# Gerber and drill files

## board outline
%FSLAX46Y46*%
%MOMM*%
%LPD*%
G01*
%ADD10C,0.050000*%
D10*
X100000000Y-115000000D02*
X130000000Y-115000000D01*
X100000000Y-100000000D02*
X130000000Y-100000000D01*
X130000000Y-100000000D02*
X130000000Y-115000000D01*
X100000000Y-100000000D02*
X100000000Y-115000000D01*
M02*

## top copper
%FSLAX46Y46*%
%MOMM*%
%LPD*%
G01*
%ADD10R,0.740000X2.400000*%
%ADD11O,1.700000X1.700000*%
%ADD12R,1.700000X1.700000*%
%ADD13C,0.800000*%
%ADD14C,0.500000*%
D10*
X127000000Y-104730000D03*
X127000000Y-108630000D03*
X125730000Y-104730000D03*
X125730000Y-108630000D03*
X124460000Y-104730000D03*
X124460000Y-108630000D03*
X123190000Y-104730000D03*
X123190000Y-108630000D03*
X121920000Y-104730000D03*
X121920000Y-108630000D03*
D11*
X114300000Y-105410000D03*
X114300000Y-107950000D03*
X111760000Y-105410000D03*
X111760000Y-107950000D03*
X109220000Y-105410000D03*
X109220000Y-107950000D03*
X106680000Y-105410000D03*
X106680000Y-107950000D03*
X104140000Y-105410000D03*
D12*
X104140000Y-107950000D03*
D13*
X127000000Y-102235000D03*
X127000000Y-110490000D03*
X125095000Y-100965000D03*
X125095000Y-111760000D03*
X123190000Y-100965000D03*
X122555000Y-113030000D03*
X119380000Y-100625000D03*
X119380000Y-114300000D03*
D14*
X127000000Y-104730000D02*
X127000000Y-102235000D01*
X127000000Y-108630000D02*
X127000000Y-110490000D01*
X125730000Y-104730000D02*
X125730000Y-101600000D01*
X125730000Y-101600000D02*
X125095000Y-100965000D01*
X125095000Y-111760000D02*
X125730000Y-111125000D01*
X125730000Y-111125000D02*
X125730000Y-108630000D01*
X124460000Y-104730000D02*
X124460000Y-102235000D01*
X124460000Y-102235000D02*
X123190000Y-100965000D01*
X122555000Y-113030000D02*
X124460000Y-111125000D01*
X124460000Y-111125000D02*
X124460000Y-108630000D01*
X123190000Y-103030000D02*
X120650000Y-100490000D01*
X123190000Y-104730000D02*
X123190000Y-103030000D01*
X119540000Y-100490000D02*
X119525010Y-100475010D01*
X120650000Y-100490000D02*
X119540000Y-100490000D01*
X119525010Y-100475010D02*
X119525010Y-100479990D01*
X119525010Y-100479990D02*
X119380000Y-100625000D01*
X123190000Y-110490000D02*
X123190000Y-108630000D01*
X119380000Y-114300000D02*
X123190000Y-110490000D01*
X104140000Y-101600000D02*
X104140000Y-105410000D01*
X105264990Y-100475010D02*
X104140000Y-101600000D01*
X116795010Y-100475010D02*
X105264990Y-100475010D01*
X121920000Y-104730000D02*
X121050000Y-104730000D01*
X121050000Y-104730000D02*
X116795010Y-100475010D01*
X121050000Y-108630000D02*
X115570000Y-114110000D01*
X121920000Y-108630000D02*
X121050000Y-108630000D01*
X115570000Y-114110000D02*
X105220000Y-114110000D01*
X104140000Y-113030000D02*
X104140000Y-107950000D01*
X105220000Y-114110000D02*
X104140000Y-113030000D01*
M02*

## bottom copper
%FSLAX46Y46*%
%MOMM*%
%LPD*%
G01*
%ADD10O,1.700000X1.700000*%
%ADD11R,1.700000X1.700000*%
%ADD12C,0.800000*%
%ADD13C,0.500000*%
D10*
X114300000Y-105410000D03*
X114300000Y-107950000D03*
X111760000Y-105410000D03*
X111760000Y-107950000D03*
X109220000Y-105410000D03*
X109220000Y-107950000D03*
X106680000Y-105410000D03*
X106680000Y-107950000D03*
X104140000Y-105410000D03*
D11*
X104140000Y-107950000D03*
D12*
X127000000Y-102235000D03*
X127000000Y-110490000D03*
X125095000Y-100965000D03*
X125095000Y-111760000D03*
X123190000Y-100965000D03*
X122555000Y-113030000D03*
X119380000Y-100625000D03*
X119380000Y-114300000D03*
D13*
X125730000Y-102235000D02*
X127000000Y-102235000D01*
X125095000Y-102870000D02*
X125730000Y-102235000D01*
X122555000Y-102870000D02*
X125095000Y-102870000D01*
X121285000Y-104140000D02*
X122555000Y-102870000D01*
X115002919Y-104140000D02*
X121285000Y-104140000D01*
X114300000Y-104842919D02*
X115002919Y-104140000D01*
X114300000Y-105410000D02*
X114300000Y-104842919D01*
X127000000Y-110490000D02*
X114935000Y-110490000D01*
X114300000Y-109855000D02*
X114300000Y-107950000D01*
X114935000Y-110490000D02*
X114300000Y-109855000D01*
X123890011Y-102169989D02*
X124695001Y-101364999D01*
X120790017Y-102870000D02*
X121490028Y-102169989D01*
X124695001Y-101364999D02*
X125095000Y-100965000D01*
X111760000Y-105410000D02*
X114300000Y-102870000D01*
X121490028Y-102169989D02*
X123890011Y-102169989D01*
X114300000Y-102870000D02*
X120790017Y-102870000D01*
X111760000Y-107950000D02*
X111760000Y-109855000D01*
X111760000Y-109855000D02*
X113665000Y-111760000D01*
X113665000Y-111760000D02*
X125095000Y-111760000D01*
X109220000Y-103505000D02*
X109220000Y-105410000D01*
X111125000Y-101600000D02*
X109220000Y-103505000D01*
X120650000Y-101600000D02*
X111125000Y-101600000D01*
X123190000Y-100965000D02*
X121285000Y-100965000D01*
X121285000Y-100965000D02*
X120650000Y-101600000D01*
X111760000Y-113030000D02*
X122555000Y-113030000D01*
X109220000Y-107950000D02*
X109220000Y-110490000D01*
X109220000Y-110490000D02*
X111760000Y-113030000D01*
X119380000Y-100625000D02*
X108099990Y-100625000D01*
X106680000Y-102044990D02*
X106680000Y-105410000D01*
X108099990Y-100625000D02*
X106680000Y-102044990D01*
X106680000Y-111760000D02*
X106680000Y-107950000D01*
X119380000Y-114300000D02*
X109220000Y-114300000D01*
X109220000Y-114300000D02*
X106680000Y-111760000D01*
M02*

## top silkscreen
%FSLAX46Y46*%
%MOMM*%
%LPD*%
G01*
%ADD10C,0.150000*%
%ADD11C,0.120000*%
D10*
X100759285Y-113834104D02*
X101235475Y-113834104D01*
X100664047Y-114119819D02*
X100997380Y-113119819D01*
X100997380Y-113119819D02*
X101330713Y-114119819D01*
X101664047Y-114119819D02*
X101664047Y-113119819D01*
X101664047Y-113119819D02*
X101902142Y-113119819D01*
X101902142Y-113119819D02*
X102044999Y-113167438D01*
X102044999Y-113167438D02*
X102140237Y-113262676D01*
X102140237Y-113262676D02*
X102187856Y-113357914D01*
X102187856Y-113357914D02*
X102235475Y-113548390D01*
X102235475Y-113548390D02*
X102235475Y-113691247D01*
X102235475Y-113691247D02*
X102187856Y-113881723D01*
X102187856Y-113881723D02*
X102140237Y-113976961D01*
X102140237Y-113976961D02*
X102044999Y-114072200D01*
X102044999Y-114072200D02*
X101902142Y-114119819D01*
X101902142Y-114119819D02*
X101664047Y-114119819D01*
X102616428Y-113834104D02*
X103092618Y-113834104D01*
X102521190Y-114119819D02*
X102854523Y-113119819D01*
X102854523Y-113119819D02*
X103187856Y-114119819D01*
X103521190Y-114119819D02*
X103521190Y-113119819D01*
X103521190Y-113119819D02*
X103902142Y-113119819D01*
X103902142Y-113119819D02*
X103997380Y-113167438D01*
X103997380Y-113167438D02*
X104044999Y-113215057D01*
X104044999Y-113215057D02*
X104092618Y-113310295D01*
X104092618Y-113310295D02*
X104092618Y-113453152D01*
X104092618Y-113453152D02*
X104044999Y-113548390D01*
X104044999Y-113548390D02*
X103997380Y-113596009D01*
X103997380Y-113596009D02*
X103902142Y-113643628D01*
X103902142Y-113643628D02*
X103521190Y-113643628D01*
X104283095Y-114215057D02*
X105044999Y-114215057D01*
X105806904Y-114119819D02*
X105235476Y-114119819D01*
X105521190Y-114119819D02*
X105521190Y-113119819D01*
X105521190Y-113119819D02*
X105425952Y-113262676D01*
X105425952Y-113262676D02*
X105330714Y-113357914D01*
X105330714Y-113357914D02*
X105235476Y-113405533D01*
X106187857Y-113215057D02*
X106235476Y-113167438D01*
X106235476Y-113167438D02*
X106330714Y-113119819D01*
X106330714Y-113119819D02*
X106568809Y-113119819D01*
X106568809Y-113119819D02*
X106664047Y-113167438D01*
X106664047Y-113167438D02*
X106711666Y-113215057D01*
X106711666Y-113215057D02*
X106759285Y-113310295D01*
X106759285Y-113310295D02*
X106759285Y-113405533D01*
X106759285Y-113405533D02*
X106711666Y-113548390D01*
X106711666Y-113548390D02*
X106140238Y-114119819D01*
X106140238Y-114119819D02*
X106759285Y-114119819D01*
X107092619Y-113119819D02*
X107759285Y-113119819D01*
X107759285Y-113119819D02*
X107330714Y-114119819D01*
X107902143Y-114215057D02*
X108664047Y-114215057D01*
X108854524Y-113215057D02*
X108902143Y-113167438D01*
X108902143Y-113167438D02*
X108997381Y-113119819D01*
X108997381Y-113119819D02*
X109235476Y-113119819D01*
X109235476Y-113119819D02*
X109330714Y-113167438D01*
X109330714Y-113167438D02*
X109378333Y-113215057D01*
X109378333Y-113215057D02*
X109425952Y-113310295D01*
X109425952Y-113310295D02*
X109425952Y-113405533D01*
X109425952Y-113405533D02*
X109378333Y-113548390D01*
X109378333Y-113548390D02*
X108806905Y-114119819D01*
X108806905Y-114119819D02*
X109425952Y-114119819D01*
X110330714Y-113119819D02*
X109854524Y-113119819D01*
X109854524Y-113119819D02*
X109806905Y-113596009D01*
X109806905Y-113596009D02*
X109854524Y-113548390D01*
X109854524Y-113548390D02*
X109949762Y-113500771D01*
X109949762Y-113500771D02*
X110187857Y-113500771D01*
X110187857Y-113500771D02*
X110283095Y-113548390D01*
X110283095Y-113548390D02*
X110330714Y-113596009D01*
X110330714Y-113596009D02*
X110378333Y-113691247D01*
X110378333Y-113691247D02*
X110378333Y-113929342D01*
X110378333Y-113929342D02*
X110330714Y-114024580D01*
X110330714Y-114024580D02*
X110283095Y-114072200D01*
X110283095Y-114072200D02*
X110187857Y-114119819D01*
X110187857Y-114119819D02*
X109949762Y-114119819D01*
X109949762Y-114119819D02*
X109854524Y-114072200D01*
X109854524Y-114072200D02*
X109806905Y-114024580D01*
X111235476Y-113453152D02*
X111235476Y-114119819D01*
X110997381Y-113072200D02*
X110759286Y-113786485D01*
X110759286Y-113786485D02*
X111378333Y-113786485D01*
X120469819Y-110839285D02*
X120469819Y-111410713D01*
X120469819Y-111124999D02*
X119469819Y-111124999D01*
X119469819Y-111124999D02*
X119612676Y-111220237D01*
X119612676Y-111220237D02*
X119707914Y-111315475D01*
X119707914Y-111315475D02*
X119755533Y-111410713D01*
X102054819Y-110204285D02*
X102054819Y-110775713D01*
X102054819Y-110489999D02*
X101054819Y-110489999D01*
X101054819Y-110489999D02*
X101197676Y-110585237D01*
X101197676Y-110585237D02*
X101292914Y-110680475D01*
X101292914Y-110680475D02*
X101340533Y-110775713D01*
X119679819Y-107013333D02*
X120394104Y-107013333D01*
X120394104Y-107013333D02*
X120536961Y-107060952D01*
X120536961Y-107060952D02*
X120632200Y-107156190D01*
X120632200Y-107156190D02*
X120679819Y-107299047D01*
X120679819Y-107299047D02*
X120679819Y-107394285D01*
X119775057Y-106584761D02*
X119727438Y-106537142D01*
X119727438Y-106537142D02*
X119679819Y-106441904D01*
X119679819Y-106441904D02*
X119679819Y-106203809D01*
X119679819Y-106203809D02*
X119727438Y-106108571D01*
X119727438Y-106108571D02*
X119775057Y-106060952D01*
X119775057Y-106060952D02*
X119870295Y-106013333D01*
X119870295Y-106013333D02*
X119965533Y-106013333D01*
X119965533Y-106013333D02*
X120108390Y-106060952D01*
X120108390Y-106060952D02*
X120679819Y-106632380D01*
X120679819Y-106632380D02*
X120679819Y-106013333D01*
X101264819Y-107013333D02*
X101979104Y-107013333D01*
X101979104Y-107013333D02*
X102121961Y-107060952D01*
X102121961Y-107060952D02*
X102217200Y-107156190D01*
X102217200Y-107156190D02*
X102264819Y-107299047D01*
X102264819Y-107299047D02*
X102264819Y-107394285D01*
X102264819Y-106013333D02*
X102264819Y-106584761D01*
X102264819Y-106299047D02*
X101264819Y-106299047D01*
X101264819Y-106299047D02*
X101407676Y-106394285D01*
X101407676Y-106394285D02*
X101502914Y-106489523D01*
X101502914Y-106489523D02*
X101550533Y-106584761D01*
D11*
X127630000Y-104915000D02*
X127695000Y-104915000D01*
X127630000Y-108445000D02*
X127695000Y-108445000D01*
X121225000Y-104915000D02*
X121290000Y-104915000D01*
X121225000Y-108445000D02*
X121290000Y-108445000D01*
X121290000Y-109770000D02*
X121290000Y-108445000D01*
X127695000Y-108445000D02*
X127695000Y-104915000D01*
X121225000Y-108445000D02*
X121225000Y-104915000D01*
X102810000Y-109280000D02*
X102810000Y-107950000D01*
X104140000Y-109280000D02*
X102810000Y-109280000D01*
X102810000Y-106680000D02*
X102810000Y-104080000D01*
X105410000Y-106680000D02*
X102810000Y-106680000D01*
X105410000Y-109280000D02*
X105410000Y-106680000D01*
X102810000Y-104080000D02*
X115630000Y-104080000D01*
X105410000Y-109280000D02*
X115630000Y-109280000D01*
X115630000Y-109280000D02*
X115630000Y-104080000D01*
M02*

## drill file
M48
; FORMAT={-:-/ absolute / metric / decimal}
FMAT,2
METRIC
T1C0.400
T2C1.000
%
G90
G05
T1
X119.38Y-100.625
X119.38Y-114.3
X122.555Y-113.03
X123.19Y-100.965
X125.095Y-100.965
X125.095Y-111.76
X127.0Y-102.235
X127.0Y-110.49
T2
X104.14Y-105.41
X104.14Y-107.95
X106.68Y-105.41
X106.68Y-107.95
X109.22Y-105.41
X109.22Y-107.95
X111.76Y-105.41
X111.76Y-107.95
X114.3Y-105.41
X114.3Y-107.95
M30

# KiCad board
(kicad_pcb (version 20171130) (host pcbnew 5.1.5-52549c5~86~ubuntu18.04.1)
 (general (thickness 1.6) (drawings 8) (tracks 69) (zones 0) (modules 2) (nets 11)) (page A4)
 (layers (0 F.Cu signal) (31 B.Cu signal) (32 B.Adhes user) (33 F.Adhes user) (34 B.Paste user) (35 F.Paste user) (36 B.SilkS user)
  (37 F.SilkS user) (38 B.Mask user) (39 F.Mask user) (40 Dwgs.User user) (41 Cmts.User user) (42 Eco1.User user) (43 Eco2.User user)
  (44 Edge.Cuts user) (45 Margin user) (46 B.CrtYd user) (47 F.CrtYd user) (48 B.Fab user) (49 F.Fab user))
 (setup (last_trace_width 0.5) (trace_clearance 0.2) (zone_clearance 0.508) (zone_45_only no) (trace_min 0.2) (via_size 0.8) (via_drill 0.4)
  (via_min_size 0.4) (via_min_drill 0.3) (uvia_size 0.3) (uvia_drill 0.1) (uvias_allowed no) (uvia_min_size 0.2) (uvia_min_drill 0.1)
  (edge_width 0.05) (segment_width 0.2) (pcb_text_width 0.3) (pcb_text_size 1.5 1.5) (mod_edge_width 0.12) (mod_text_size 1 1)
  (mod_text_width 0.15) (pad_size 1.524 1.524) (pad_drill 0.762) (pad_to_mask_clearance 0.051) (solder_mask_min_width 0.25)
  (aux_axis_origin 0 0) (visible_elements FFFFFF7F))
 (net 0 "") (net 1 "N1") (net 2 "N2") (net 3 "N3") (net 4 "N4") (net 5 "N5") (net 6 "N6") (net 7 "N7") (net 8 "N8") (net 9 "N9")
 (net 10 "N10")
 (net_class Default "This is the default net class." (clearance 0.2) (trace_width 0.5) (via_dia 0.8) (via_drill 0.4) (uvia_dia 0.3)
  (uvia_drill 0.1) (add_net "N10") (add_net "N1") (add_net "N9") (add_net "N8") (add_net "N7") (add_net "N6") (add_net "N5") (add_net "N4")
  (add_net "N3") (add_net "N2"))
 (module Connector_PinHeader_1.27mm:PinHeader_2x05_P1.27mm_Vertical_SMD (layer F.Cu) (at 124.46 106.68 90)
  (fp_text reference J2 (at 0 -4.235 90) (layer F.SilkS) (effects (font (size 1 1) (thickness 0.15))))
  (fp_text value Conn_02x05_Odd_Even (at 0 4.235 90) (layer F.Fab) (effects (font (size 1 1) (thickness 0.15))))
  (fp_line (start 1.765 3.17) (end 1.765 3.235) (layer F.SilkS) (width 0.12))
  (fp_line (start -1.765 3.17) (end -1.765 3.235) (layer F.SilkS) (width 0.12))
  (fp_line (start 1.765 -3.235) (end 1.765 -3.17) (layer F.SilkS) (width 0.12))
  (fp_line (start -1.765 -3.235) (end -1.765 -3.17) (layer F.SilkS) (width 0.12))
  (fp_line (start -3.09 -3.17) (end -1.765 -3.17) (layer F.SilkS) (width 0.12))
  (fp_line (start -1.765 3.235) (end 1.765 3.235) (layer F.SilkS) (width 0.12))
  (fp_line (start -1.765 -3.235) (end 1.765 -3.235) (layer F.SilkS) (width 0.12))
  (pad 10 smd rect (at 1.95 2.54 90) (size 2.4 0.74) (layers F.Cu F.Paste F.Mask) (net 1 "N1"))
  (pad 9 smd rect (at -1.95 2.54 90) (size 2.4 0.74) (layers F.Cu F.Paste F.Mask) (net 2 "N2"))
  (pad 8 smd rect (at 1.95 1.27 90) (size 2.4 0.74) (layers F.Cu F.Paste F.Mask) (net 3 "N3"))
  (pad 7 smd rect (at -1.95 1.27 90) (size 2.4 0.74) (layers F.Cu F.Paste F.Mask) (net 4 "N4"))
  (pad 6 smd rect (at 1.95 0 90) (size 2.4 0.74) (layers F.Cu F.Paste F.Mask) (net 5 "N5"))
  (pad 5 smd rect (at -1.95 0 90) (size 2.4 0.74) (layers F.Cu F.Paste F.Mask) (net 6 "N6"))
  (pad 4 smd rect (at 1.95 -1.27 90) (size 2.4 0.74) (layers F.Cu F.Paste F.Mask) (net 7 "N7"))
  (pad 3 smd rect (at -1.95 -1.27 90) (size 2.4 0.74) (layers F.Cu F.Paste F.Mask) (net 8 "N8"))
  (pad 2 smd rect (at 1.95 -2.54 90) (size 2.4 0.74) (layers F.Cu F.Paste F.Mask) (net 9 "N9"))
  (pad 1 smd rect (at -1.95 -2.54 90) (size 2.4 0.74) (layers F.Cu F.Paste F.Mask) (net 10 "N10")))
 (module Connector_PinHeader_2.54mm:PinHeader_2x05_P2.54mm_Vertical (layer F.Cu) (at 104.14 107.95 90)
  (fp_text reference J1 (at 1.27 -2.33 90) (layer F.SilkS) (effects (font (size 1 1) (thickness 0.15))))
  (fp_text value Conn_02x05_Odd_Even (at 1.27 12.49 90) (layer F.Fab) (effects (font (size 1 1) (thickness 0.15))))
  (fp_line (start -1.33 -1.33) (end 0 -1.33) (layer F.SilkS) (width 0.12))
  (fp_line (start -1.33 0) (end -1.33 -1.33) (layer F.SilkS) (width 0.12))
  (fp_line (start 1.27 -1.33) (end 3.87 -1.33) (layer F.SilkS) (width 0.12))
  (fp_line (start 1.27 1.27) (end 1.27 -1.33) (layer F.SilkS) (width 0.12))
  (fp_line (start -1.33 1.27) (end 1.27 1.27) (layer F.SilkS) (width 0.12))
  (fp_line (start 3.87 -1.33) (end 3.87 11.49) (layer F.SilkS) (width 0.12))
  (fp_line (start -1.33 1.27) (end -1.33 11.49) (layer F.SilkS) (width 0.12))
  (fp_line (start -1.33 11.49) (end 3.87 11.49) (layer F.SilkS) (width 0.12))
  (pad 10 thru_hole oval (at 2.54 10.16 90) (size 1.7 1.7) (drill 1) (layers *.Cu *.Mask) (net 1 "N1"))
  (pad 9 thru_hole oval (at 0 10.16 90) (size 1.7 1.7) (drill 1) (layers *.Cu *.Mask) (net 2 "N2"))
  (pad 8 thru_hole oval (at 2.54 7.62 90) (size 1.7 1.7) (drill 1) (layers *.Cu *.Mask) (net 3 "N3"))
  (pad 7 thru_hole oval (at 0 7.62 90) (size 1.7 1.7) (drill 1) (layers *.Cu *.Mask) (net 4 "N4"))
  (pad 6 thru_hole oval (at 2.54 5.08 90) (size 1.7 1.7) (drill 1) (layers *.Cu *.Mask) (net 5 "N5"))
  (pad 5 thru_hole oval (at 0 5.08 90) (size 1.7 1.7) (drill 1) (layers *.Cu *.Mask) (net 6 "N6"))
  (pad 4 thru_hole oval (at 2.54 2.54 90) (size 1.7 1.7) (drill 1) (layers *.Cu *.Mask) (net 7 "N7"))
  (pad 3 thru_hole oval (at 0 2.54 90) (size 1.7 1.7) (drill 1) (layers *.Cu *.Mask) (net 8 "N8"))
  (pad 2 thru_hole oval (at 2.54 0 90) (size 1.7 1.7) (drill 1) (layers *.Cu *.Mask) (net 9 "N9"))
  (pad 1 thru_hole rect (at 0 0 90) (size 1.7 1.7) (drill 1) (layers *.Cu *.Mask) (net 10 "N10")))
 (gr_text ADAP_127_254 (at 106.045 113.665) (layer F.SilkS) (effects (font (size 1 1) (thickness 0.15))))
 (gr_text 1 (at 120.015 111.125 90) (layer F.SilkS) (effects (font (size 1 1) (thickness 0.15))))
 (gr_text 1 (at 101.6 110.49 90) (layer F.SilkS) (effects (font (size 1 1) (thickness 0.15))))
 (gr_line (start 100 115) (end 130 115) (layer Edge.Cuts) (width 0.05))
 (gr_line (start 100 100) (end 130 100) (layer Edge.Cuts) (width 0.05))
 (gr_line (start 130 100) (end 130 115) (layer Edge.Cuts) (width 0.05))
 (gr_line (start 100 100) (end 100 115) (layer Edge.Cuts) (width 0.05))
 (segment (start 127 104.73) (end 127 102.235) (width 0.5) (layer F.Cu) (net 1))
 (via (at 127 102.235) (size 0.8) (drill 0.4) (layers F.Cu B.Cu) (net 1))
 (segment (start 125.73 102.235) (end 127 102.235) (width 0.5) (layer B.Cu) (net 1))
 (segment (start 125.095 102.87) (end 125.73 102.235) (width 0.5) (layer B.Cu) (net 1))
 (segment (start 122.555 102.87) (end 125.095 102.87) (width 0.5) (layer B.Cu) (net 1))
 (segment (start 121.285 104.14) (end 122.555 102.87) (width 0.5) (layer B.Cu) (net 1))
 (segment (start 115.002919 104.14) (end 121.285 104.14) (width 0.5) (layer B.Cu) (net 1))
 (segment (start 114.3 104.842919) (end 115.002919 104.14) (width 0.5) (layer B.Cu) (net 1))
 (segment (start 114.3 105.41) (end 114.3 104.842919) (width 0.5) (layer B.Cu) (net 1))
 (segment (start 127 108.63) (end 127 110.49) (width 0.5) (layer F.Cu) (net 2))
 (via (at 127 110.49) (size 0.8) (drill 0.4) (layers F.Cu B.Cu) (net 2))
 (segment (start 127 110.49) (end 114.935 110.49) (width 0.5) (layer B.Cu) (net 2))
 (segment (start 114.3 109.855) (end 114.3 107.95) (width 0.5) (layer B.Cu) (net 2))
 (segment (start 114.935 110.49) (end 114.3 109.855) (width 0.5) (layer B.Cu) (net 2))
 (segment (start 125.73 104.73) (end 125.73 101.6) (width 0.5) (layer F.Cu) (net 3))
 (segment (start 125.73 101.6) (end 125.095 100.965) (width 0.5) (layer F.Cu) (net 3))
 (via (at 125.095 100.965) (size 0.8) (drill 0.4) (layers F.Cu B.Cu) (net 3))
 (segment (start 123.890011 102.169989) (end 124.695001 101.364999) (width 0.5) (layer B.Cu) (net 3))
 (segment (start 120.790017 102.87) (end 121.490028 102.169989) (width 0.5) (layer B.Cu) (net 3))
 (segment (start 124.695001 101.364999) (end 125.095 100.965) (width 0.5) (layer B.Cu) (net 3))
 (segment (start 111.76 105.41) (end 114.3 102.87) (width 0.5) (layer B.Cu) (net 3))
 (segment (start 121.490028 102.169989) (end 123.890011 102.169989) (width 0.5) (layer B.Cu) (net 3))
 (segment (start 114.3 102.87) (end 120.790017 102.87) (width 0.5) (layer B.Cu) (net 3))
 (segment (start 111.76 107.95) (end 111.76 109.855) (width 0.5) (layer B.Cu) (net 4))
 (segment (start 111.76 109.855) (end 113.665 111.76) (width 0.5) (layer B.Cu) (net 4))
 (segment (start 113.665 111.76) (end 125.095 111.76) (width 0.5) (layer B.Cu) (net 4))
 (via (at 125.095 111.76) (size 0.8) (drill 0.4) (layers F.Cu B.Cu) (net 4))
 (segment (start 125.095 111.76) (end 125.73 111.125) (width 0.5) (layer F.Cu) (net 4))
 (segment (start 125.73 111.125) (end 125.73 108.63) (width 0.5) (layer F.Cu) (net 4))
 (segment (start 124.46 104.73) (end 124.46 102.235) (width 0.5) (layer F.Cu) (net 5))
 (segment (start 124.46 102.235) (end 123.19 100.965) (width 0.5) (layer F.Cu) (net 5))
 (via (at 123.19 100.965) (size 0.8) (drill 0.4) (layers F.Cu B.Cu) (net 5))
 (segment (start 109.22 103.505) (end 109.22 105.41) (width 0.5) (layer B.Cu) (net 5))
 (segment (start 111.125 101.6) (end 109.22 103.505) (width 0.5) (layer B.Cu) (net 5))
 (segment (start 120.65 101.6) (end 111.125 101.6) (width 0.5) (layer B.Cu) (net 5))
 (segment (start 123.19 100.965) (end 121.285 100.965) (width 0.5) (layer B.Cu) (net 5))
 (segment (start 121.285 100.965) (end 120.65 101.6) (width 0.5) (layer B.Cu) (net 5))
 (via (at 122.555 113.03) (size 0.8) (drill 0.4) (layers F.Cu B.Cu) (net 6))
 (segment (start 122.555 113.03) (end 124.46 111.125) (width 0.5) (layer F.Cu) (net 6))
 (segment (start 124.46 111.125) (end 124.46 108.63) (width 0.5) (layer F.Cu) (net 6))
 (segment (start 111.76 113.03) (end 122.555 113.03) (width 0.5) (layer B.Cu) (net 6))
 (segment (start 109.22 107.95) (end 109.22 110.49) (width 0.5) (layer B.Cu) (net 6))
 (segment (start 109.22 110.49) (end 111.76 113.03) (width 0.5) (layer B.Cu) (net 6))
 (segment (start 123.19 103.03) (end 120.65 100.49) (width 0.5) (layer F.Cu) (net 7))
 (segment (start 123.19 104.73) (end 123.19 103.03) (width 0.5) (layer F.Cu) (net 7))
 (segment (start 119.54 100.49) (end 119.52501 100.47501) (width 0.5) (layer F.Cu) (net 7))
 (segment (start 120.65 100.49) (end 119.54 100.49) (width 0.5) (layer F.Cu) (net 7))
 (via (at 119.38 100.625) (size 0.8) (drill 0.4) (layers F.Cu B.Cu) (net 7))
 (segment (start 119.52501 100.47501) (end 119.52501 100.47999) (width 0.5) (layer F.Cu) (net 7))
 (segment (start 119.52501 100.47999) (end 119.38 100.625) (width 0.5) (layer F.Cu) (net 7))
 (segment (start 119.38 100.625) (end 108.09999 100.625) (width 0.5) (layer B.Cu) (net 7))
 (segment (start 106.68 102.04499) (end 106.68 105.41) (width 0.5) (layer B.Cu) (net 7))
 (segment (start 108.09999 100.625) (end 106.68 102.04499) (width 0.5) (layer B.Cu) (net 7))
 (via (at 119.38 114.3) (size 0.8) (drill 0.4) (layers F.Cu B.Cu) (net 8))
 (segment (start 123.19 110.49) (end 123.19 108.63) (width 0.5) (layer F.Cu) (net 8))
 (segment (start 119.38 114.3) (end 123.19 110.49) (width 0.5) (layer F.Cu) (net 8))
 (segment (start 106.68 111.76) (end 106.68 107.95) (width 0.5) (layer B.Cu) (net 8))
 (segment (start 119.38 114.3) (end 109.22 114.3) (width 0.5) (layer B.Cu) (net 8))
 (segment (start 109.22 114.3) (end 106.68 111.76) (width 0.5) (layer B.Cu) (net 8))
 (segment (start 104.14 101.6) (end 104.14 105.41) (width 0.5) (layer F.Cu) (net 9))
 (segment (start 105.26499 100.47501) (end 104.14 101.6) (width 0.5) (layer F.Cu) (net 9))
 (segment (start 116.79501 100.47501) (end 105.26499 100.47501) (width 0.5) (layer F.Cu) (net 9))
 (segment (start 121.92 104.73) (end 121.05 104.73) (width 0.5) (layer F.Cu) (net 9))
 (segment (start 121.05 104.73) (end 116.79501 100.47501) (width 0.5) (layer F.Cu) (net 9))
 (segment (start 121.05 108.63) (end 115.57 114.11) (width 0.5) (layer F.Cu) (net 10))
 (segment (start 121.92 108.63) (end 121.05 108.63) (width 0.5) (layer F.Cu) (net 10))
 (segment (start 115.57 114.11) (end 105.22 114.11) (width 0.5) (layer F.Cu) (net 10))
 (segment (start 104.14 113.03) (end 104.14 107.95) (width 0.5) (layer F.Cu) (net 10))
 (segment (start 105.22 114.11) (end 104.14 113.03) (width 0.5) (layer F.Cu) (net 10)))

